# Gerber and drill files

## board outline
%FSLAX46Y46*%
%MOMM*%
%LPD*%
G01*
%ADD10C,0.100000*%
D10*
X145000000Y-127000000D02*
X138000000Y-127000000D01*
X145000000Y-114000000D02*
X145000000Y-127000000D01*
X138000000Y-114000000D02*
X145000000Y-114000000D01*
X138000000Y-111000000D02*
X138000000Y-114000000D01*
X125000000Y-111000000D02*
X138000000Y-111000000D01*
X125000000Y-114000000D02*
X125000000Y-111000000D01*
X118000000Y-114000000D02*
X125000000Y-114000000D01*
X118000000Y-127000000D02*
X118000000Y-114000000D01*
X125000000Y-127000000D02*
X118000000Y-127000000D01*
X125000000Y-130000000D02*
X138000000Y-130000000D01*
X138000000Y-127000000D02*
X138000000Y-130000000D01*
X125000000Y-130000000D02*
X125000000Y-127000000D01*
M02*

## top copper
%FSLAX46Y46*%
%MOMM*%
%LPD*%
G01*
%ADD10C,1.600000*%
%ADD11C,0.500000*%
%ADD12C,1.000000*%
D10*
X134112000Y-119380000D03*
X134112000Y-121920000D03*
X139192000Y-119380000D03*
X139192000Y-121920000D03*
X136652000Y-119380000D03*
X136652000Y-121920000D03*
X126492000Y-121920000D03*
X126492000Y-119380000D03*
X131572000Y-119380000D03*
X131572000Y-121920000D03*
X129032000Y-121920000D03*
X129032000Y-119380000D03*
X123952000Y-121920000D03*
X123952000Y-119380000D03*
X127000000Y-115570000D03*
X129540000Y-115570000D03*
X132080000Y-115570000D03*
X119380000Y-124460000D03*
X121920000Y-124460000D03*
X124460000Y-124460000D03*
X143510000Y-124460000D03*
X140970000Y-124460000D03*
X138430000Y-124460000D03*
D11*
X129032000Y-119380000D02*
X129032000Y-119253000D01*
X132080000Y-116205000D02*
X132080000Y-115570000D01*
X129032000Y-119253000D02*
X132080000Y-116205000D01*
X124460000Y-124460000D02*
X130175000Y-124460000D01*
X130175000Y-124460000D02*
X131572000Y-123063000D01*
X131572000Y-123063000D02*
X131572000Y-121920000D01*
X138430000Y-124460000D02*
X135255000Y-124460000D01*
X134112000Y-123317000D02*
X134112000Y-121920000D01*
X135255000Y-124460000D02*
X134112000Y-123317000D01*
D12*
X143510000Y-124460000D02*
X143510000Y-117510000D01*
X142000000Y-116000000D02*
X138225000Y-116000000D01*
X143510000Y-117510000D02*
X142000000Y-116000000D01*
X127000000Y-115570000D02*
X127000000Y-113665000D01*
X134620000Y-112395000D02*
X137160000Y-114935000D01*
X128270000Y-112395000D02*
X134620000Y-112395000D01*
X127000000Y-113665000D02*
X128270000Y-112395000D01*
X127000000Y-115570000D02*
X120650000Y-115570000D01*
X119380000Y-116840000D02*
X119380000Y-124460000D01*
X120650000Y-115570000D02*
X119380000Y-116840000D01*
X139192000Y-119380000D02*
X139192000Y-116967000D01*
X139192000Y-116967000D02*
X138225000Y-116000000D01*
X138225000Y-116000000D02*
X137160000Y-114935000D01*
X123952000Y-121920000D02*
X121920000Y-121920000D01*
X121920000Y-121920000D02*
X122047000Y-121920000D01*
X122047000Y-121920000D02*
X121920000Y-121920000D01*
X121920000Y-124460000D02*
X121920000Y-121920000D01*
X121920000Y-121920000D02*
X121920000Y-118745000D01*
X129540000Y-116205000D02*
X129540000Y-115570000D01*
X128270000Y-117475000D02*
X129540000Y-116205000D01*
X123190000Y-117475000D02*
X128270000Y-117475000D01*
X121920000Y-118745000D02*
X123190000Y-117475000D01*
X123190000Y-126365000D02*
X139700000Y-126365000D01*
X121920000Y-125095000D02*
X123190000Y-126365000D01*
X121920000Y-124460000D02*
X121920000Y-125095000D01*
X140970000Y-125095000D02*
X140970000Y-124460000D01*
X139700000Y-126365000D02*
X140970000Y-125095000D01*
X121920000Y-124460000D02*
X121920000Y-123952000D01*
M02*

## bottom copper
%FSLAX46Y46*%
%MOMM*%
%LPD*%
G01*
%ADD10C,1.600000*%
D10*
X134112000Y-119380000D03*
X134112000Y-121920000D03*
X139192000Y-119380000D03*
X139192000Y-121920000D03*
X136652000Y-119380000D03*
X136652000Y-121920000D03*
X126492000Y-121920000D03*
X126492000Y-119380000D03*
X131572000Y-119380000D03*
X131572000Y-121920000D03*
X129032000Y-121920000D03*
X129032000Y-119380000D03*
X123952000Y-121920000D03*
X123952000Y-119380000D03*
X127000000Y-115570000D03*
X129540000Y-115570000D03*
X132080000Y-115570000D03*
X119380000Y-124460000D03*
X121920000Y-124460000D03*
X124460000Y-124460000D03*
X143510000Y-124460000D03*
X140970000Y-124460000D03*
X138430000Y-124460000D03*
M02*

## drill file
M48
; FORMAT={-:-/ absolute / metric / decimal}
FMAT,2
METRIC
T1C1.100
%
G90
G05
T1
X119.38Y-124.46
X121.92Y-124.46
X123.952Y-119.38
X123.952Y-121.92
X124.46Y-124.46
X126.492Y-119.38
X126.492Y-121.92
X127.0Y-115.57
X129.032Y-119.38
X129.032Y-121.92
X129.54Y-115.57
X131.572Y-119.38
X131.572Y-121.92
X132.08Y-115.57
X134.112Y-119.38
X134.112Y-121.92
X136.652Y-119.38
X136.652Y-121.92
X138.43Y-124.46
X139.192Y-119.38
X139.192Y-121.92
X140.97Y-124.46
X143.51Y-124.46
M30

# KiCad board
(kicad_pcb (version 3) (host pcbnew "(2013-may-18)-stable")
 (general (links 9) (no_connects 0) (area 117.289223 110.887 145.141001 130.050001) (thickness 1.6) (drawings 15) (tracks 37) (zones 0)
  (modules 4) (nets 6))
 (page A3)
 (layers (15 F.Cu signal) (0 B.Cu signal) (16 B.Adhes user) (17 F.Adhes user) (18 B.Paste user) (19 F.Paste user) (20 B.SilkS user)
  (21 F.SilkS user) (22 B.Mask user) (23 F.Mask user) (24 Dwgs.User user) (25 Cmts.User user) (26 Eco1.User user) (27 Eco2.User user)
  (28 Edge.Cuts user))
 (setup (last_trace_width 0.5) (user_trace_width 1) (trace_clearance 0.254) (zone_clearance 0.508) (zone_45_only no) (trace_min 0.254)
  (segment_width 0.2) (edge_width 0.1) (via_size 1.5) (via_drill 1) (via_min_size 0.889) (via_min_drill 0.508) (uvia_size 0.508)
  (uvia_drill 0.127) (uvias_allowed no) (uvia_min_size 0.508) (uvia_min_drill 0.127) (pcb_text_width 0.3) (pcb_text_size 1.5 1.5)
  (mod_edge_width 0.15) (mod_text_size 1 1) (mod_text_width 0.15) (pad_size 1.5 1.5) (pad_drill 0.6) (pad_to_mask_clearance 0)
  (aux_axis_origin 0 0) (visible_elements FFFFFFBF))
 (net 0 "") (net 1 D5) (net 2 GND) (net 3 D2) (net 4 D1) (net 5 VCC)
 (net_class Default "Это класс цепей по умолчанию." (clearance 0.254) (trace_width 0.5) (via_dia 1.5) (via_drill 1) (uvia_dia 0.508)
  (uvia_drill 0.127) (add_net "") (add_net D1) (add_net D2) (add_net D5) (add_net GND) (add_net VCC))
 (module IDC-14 (layer B.Cu) (at 131.572 120.65)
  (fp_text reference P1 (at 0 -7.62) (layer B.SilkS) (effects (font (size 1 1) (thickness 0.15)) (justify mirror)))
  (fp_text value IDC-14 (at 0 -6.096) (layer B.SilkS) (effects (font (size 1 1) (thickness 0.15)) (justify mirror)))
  (pad 5 thru_hole circle (at 2.54 -1.27) (size 1.6 1.6) (drill 1.1) (layers *.Cu *.Mask B.SilkS))
  (pad 6 thru_hole circle (at 2.54 1.27) (size 1.6 1.6) (drill 1.1) (layers *.Cu *.Mask B.SilkS) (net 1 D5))
  (pad 1 thru_hole circle (at 7.62 -1.27) (size 1.6 1.6) (drill 1.1) (layers *.Cu *.Mask B.SilkS) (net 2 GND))
  (pad 2 thru_hole circle (at 7.62 1.27) (size 1.6 1.6) (drill 1.1) (layers *.Cu *.Mask B.SilkS))
  (pad 3 thru_hole circle (at 5.08 -1.27) (size 1.6 1.6) (drill 1.1) (layers *.Cu *.Mask B.SilkS))
  (pad 4 thru_hole circle (at 5.08 1.27) (size 1.6 1.6) (drill 1.1) (layers *.Cu *.Mask B.SilkS))
  (pad 12 thru_hole circle (at -5.08 1.27) (size 1.6 1.6) (drill 1.1) (layers *.Cu *.Mask B.SilkS))
  (pad 11 thru_hole circle (at -5.08 -1.27) (size 1.6 1.6) (drill 1.1) (layers *.Cu *.Mask B.SilkS))
  (pad 7 thru_hole circle (at 0 -1.27) (size 1.6 1.6) (drill 1.1) (layers *.Cu *.Mask B.SilkS))
  (pad 8 thru_hole circle (at 0 1.27) (size 1.6 1.6) (drill 1.1) (layers *.Cu *.Mask B.SilkS) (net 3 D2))
  (pad 10 thru_hole circle (at -2.54 1.27) (size 1.6 1.6) (drill 1.1) (layers *.Cu *.Mask B.SilkS))
  (pad 9 thru_hole circle (at -2.54 -1.27) (size 1.6 1.6) (drill 1.1) (layers *.Cu *.Mask B.SilkS) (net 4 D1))
  (pad 14 thru_hole circle (at -7.62 1.27) (size 1.6 1.6) (drill 1.1) (layers *.Cu *.Mask B.SilkS) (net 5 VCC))
  (pad 13 thru_hole circle (at -7.62 -1.27) (size 1.6 1.6) (drill 1.1) (layers *.Cu *.Mask B.SilkS)))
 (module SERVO (layer F.Cu) (at 129.54 115.57)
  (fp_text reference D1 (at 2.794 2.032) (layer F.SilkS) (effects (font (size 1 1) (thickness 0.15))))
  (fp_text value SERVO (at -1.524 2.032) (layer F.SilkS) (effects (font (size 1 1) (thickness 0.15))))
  (pad 1 thru_hole circle (at -2.54 0) (size 1.6 1.6) (drill 1.1) (layers *.Cu *.Mask F.SilkS) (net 2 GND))
  (pad 2 thru_hole circle (at 0 0) (size 1.6 1.6) (drill 1.1) (layers *.Cu *.Mask F.SilkS) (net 5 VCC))
  (pad 3 thru_hole circle (at 2.54 0) (size 1.6 1.6) (drill 1.1) (layers *.Cu *.Mask F.SilkS) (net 4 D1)))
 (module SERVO (layer F.Cu) (at 121.92 124.46)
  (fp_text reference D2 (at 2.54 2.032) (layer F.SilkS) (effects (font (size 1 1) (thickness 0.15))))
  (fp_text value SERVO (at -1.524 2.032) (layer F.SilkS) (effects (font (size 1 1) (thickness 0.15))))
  (pad 1 thru_hole circle (at -2.54 0) (size 1.6 1.6) (drill 1.1) (layers *.Cu *.Mask F.SilkS) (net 2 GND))
  (pad 2 thru_hole circle (at 0 0) (size 1.6 1.6) (drill 1.1) (layers *.Cu *.Mask F.SilkS) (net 5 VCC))
  (pad 3 thru_hole circle (at 2.54 0) (size 1.6 1.6) (drill 1.1) (layers *.Cu *.Mask F.SilkS) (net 3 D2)))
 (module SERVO (layer F.Cu) (at 140.97 124.46 180)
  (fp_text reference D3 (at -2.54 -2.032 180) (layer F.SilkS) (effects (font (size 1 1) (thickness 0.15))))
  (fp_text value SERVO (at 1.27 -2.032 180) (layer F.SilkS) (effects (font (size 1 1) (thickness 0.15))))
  (pad 1 thru_hole circle (at -2.54 0 180) (size 1.6 1.6) (drill 1.1) (layers *.Cu *.Mask F.SilkS) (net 2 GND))
  (pad 2 thru_hole circle (at 0 0 180) (size 1.6 1.6) (drill 1.1) (layers *.Cu *.Mask F.SilkS) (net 5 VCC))
  (pad 3 thru_hole circle (at 2.54 0 180) (size 1.6 1.6) (drill 1.1) (layers *.Cu *.Mask F.SilkS) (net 1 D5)))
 (gr_line (start 145 127) (end 138 127) (angle 90) (layer Edge.Cuts) (width 0.1))
 (gr_line (start 145 114) (end 145 127) (angle 90) (layer Edge.Cuts) (width 0.1))
 (gr_line (start 138 114) (end 145 114) (angle 90) (layer Edge.Cuts) (width 0.1))
 (gr_line (start 138 111) (end 138 114) (angle 90) (layer Edge.Cuts) (width 0.1))
 (gr_line (start 125 111) (end 138 111) (angle 90) (layer Edge.Cuts) (width 0.1))
 (gr_line (start 125 114) (end 125 111) (angle 90) (layer Edge.Cuts) (width 0.1))
 (gr_line (start 118 114) (end 125 114) (angle 90) (layer Edge.Cuts) (width 0.1))
 (gr_line (start 118 127) (end 118 114) (angle 90) (layer Edge.Cuts) (width 0.1))
 (gr_line (start 125 127) (end 118 127) (angle 90) (layer Edge.Cuts) (width 0.1))
 (gr_line (start 125 130) (end 138 130) (angle 90) (layer Edge.Cuts) (width 0.1))
 (gr_line (start 138 127) (end 138 130) (angle 90) (layer Edge.Cuts) (width 0.1))
 (gr_line (start 125 130) (end 125 127) (angle 90) (layer Edge.Cuts) (width 0.1))
 (segment (start 129.032 119.38) (end 129.032 119.253) (width 0.5) (layer F.Cu) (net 4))
 (segment (start 132.08 116.205) (end 132.08 115.57) (width 0.5) (layer F.Cu) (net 4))
 (segment (start 129.032 119.253) (end 132.08 116.205) (width 0.5) (layer F.Cu) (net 4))
 (segment (start 124.46 124.46) (end 130.175 124.46) (width 0.5) (layer F.Cu) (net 3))
 (segment (start 130.175 124.46) (end 131.572 123.063) (width 0.5) (layer F.Cu) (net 3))
 (segment (start 131.572 123.063) (end 131.572 121.92) (width 0.5) (layer F.Cu) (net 3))
 (segment (start 138.43 124.46) (end 135.255 124.46) (width 0.5) (layer F.Cu) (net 1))
 (segment (start 134.112 123.317) (end 134.112 121.92) (width 0.5) (layer F.Cu) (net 1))
 (segment (start 135.255 124.46) (end 134.112 123.317) (width 0.5) (layer F.Cu) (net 1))
 (segment (start 143.51 124.46) (end 143.51 117.51) (width 1) (layer F.Cu) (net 2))
 (segment (start 142 116) (end 138.225 116) (width 1) (layer F.Cu) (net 2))
 (segment (start 143.51 117.51) (end 142 116) (width 1) (layer F.Cu) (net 2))
 (segment (start 127 115.57) (end 127 113.665) (width 1) (layer F.Cu) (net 2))
 (segment (start 134.62 112.395) (end 137.16 114.935) (width 1) (layer F.Cu) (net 2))
 (segment (start 128.27 112.395) (end 134.62 112.395) (width 1) (layer F.Cu) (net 2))
 (segment (start 127 113.665) (end 128.27 112.395) (width 1) (layer F.Cu) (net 2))
 (segment (start 127 115.57) (end 120.65 115.57) (width 1) (layer F.Cu) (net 2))
 (segment (start 119.38 116.84) (end 119.38 124.46) (width 1) (layer F.Cu) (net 2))
 (segment (start 120.65 115.57) (end 119.38 116.84) (width 1) (layer F.Cu) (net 2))
 (segment (start 139.192 119.38) (end 139.192 116.967) (width 1) (layer F.Cu) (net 2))
 (segment (start 139.192 116.967) (end 138.225 116) (width 1) (layer F.Cu) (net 2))
 (segment (start 138.225 116) (end 137.16 114.935) (width 1) (layer F.Cu) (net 2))
 (segment (start 123.952 121.92) (end 121.92 121.92) (width 1) (layer F.Cu) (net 5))
 (segment (start 121.92 121.92) (end 122.047 121.92) (width 1) (layer F.Cu) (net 5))
 (segment (start 122.047 121.92) (end 121.92 121.92) (width 1) (layer F.Cu) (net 5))
 (segment (start 121.92 124.46) (end 121.92 121.92) (width 1) (layer F.Cu) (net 5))
 (segment (start 121.92 121.92) (end 121.92 118.745) (width 1) (layer F.Cu) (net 5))
 (segment (start 129.54 116.205) (end 129.54 115.57) (width 1) (layer F.Cu) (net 5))
 (segment (start 128.27 117.475) (end 129.54 116.205) (width 1) (layer F.Cu) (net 5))
 (segment (start 123.19 117.475) (end 128.27 117.475) (width 1) (layer F.Cu) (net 5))
 (segment (start 121.92 118.745) (end 123.19 117.475) (width 1) (layer F.Cu) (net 5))
 (segment (start 123.19 126.365) (end 139.7 126.365) (width 1) (layer F.Cu) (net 5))
 (segment (start 121.92 125.095) (end 123.19 126.365) (width 1) (layer F.Cu) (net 5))
 (segment (start 121.92 124.46) (end 121.92 125.095) (width 1) (layer F.Cu) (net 5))
 (segment (start 140.97 125.095) (end 140.97 124.46) (width 1) (layer F.Cu) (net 5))
 (segment (start 139.7 126.365) (end 140.97 125.095) (width 1) (layer F.Cu) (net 5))
 (segment (start 121.92 124.46) (end 121.92 123.952) (width 1) (layer F.Cu) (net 5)))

